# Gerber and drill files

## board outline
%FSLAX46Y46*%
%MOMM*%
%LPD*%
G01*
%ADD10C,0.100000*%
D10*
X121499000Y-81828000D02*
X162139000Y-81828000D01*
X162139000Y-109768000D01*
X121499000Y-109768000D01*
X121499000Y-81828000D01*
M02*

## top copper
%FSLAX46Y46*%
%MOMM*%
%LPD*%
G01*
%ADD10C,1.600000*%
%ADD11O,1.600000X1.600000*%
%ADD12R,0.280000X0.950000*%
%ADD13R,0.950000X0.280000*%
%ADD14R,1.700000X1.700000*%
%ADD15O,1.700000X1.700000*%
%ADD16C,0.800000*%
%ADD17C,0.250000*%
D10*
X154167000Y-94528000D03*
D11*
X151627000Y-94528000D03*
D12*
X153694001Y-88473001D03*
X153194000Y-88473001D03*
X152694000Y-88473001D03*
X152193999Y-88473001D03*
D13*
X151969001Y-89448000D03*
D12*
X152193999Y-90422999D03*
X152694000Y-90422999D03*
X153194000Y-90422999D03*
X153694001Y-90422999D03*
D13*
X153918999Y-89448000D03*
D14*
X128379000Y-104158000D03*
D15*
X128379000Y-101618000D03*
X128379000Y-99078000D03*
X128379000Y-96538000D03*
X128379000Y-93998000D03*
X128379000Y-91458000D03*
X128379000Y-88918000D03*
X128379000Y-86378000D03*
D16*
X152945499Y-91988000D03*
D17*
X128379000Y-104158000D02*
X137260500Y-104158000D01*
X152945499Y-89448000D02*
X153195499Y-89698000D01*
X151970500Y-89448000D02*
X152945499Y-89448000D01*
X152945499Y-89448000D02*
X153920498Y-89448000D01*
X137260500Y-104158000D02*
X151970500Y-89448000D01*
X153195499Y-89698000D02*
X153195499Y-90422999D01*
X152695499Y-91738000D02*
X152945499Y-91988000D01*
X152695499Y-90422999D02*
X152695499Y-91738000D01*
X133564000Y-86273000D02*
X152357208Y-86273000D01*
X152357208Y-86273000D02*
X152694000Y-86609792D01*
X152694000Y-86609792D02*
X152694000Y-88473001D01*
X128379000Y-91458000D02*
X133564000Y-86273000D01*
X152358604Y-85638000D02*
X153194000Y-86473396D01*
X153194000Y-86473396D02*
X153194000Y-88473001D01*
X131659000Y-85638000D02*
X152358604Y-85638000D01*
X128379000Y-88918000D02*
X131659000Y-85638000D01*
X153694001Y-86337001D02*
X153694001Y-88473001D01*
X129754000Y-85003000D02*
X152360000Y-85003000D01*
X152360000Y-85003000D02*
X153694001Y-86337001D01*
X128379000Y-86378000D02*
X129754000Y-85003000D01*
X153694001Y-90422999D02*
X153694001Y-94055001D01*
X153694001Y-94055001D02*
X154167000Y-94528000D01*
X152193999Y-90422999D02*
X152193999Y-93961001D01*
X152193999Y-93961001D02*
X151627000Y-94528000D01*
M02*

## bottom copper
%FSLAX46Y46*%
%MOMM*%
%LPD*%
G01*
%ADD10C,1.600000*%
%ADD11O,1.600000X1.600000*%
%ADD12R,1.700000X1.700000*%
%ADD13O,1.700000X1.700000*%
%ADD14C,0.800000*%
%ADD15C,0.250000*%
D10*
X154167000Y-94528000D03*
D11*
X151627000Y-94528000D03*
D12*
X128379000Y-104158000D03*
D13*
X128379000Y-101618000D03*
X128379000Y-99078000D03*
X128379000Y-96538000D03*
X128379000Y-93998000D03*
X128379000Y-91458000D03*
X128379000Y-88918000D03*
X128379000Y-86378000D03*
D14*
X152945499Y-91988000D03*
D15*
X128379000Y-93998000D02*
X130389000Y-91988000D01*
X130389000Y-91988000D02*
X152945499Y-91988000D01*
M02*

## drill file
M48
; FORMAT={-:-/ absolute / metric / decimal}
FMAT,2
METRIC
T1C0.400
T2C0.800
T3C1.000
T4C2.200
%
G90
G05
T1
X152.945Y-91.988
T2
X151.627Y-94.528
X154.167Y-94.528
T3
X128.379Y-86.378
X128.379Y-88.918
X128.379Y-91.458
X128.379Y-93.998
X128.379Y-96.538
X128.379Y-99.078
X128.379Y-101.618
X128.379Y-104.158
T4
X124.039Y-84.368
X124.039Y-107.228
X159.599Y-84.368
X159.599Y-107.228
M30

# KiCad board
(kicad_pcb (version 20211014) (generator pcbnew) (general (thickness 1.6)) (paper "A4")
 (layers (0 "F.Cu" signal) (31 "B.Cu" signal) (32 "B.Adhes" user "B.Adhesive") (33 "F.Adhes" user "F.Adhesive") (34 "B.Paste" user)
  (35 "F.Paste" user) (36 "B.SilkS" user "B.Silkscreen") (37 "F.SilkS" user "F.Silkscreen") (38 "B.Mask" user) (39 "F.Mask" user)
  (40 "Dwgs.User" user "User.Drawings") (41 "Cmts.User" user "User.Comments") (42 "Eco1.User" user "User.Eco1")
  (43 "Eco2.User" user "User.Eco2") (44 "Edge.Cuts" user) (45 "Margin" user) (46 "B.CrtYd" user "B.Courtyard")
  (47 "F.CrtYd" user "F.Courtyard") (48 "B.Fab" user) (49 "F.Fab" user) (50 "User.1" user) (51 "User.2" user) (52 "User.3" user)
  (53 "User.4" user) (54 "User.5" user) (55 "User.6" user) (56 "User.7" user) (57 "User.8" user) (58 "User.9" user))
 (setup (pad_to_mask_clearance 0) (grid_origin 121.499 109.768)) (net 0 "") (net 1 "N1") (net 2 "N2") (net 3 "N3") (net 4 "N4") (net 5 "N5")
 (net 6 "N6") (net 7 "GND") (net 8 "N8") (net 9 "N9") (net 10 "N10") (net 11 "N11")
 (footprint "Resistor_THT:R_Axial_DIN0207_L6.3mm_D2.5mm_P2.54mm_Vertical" (layer "F.Cu") (at 154.167 94.528 180)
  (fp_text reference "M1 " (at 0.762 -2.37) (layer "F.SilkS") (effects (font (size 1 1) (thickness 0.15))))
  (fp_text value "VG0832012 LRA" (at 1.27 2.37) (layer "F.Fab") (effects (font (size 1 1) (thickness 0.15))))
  (pad "1" thru_hole circle (at 0 0 180) (size 1.6 1.6) (drill 0.8) (layers *.Cu *.Mask) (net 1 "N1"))
  (pad "2" thru_hole oval (at 2.54 0 180) (size 1.6 1.6) (drill 0.8) (layers *.Cu *.Mask) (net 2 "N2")))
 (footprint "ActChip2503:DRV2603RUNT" (layer "F.Cu") (at 152.944 89.448 -90)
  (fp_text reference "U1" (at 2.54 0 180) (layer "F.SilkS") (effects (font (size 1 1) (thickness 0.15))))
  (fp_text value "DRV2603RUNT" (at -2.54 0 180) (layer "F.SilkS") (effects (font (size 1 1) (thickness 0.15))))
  (pad "1" smd rect (at -0.974999 -0.750001) (size 0.28 0.95) (layers "F.Cu" "F.Paste" "F.Mask") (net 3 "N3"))
  (pad "2" smd rect (at -0.974999 -0.25) (size 0.28 0.95) (layers "F.Cu" "F.Paste" "F.Mask") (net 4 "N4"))
  (pad "3" smd rect (at -0.974999 0.25) (size 0.28 0.95) (layers "F.Cu" "F.Paste" "F.Mask") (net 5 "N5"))
  (pad "4" smd rect (at -0.974999 0.750001) (size 0.28 0.95) (layers "F.Cu" "F.Paste" "F.Mask") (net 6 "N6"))
  (pad "5" smd rect (at 0 0.974999 270) (size 0.28 0.95) (layers "F.Cu" "F.Paste" "F.Mask") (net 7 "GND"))
  (pad "6" smd rect (at 0.974999 0.750001) (size 0.28 0.95) (layers "F.Cu" "F.Paste" "F.Mask") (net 2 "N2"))
  (pad "7" smd rect (at 0.974999 0.25) (size 0.28 0.95) (layers "F.Cu" "F.Paste" "F.Mask") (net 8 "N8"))
  (pad "8" smd rect (at 0.974999 -0.25) (size 0.28 0.95) (layers "F.Cu" "F.Paste" "F.Mask") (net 7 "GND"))
  (pad "9" smd rect (at 0.974999 -0.750001) (size 0.28 0.95) (layers "F.Cu" "F.Paste" "F.Mask") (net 1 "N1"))
  (pad "10" smd rect (at 0 -0.974999 270) (size 0.28 0.95) (layers "F.Cu" "F.Paste" "F.Mask") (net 7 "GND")))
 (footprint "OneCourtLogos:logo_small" (layer "F.Cu") (at 141.819 94.528)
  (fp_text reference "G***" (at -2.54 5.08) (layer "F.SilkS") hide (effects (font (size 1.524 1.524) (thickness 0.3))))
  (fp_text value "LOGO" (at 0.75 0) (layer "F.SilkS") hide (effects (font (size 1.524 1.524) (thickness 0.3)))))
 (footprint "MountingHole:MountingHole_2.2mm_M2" (layer "F.Cu") (at 159.599 84.368)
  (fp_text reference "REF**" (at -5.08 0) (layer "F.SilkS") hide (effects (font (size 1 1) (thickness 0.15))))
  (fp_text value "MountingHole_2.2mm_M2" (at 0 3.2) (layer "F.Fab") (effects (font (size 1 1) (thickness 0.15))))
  (pad "" np_thru_hole circle (at 0 0) (size 2.2 2.2) (drill 2.2) (layers *.Cu *.Mask)))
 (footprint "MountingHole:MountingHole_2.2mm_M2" (layer "F.Cu") (at 124.039 107.228)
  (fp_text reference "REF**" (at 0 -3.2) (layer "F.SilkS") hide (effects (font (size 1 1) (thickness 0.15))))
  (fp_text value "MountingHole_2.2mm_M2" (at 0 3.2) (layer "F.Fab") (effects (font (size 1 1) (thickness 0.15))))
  (pad "" np_thru_hole circle (at 0 0) (size 2.2 2.2) (drill 2.2) (layers *.Cu *.Mask)))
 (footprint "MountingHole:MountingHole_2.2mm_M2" (layer "F.Cu") (at 124.039 84.368)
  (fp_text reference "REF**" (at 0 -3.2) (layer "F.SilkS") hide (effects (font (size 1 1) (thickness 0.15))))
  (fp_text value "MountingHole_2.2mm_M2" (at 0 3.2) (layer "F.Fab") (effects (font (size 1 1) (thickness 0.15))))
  (pad "" np_thru_hole circle (at 0 0) (size 2.2 2.2) (drill 2.2) (layers *.Cu *.Mask)))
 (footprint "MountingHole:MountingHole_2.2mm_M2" (layer "F.Cu") (at 159.599 107.228)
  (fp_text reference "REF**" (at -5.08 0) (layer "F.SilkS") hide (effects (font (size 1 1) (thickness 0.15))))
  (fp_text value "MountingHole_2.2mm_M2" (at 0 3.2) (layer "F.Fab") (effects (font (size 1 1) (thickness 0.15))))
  (pad "" np_thru_hole circle (at 0 0) (size 2.2 2.2) (drill 2.2) (layers *.Cu *.Mask)))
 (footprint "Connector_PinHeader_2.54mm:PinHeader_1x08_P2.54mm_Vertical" (layer "F.Cu") (at 128.379 104.158 180)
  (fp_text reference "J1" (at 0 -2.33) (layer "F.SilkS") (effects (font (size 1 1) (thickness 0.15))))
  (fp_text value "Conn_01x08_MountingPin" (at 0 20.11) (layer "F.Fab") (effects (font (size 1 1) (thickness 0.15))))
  (pad "1" thru_hole rect (at 0 0 180) (size 1.7 1.7) (drill 1) (layers *.Cu *.Mask) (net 7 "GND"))
  (pad "2" thru_hole oval (at 0 2.54 180) (size 1.7 1.7) (drill 1) (layers *.Cu *.Mask) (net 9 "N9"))
  (pad "3" thru_hole oval (at 0 5.08 180) (size 1.7 1.7) (drill 1) (layers *.Cu *.Mask) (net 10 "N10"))
  (pad "4" thru_hole oval (at 0 7.62 180) (size 1.7 1.7) (drill 1) (layers *.Cu *.Mask) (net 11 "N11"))
  (pad "5" thru_hole oval (at 0 10.16 180) (size 1.7 1.7) (drill 1) (layers *.Cu *.Mask) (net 8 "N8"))
  (pad "6" thru_hole oval (at 0 12.7 180) (size 1.7 1.7) (drill 1) (layers *.Cu *.Mask) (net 5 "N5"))
  (pad "7" thru_hole oval (at 0 15.24 180) (size 1.7 1.7) (drill 1) (layers *.Cu *.Mask) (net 4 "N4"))
  (pad "8" thru_hole oval (at 0 17.78 180) (size 1.7 1.7) (drill 1) (layers *.Cu *.Mask) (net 3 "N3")))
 (gr_rect (start 121.499 81.828) (end 162.139 109.768) (layer "Edge.Cuts") (width 0.1) (fill none))
 (segment (start 128.379 104.158) (end 137.2605 104.158) (width 0.25) (layer "F.Cu") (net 7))
 (segment (start 152.945499 89.448) (end 153.195499 89.698) (width 0.25) (layer "F.Cu") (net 7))
 (segment (start 151.9705 89.448) (end 152.945499 89.448) (width 0.25) (layer "F.Cu") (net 7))
 (segment (start 152.945499 89.448) (end 153.920498 89.448) (width 0.25) (layer "F.Cu") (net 7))
 (segment (start 137.2605 104.158) (end 151.9705 89.448) (width 0.25) (layer "F.Cu") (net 7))
 (segment (start 153.195499 89.698) (end 153.195499 90.422999) (width 0.25) (layer "F.Cu") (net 7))
 (segment (start 152.695499 91.738) (end 152.945499 91.988) (width 0.25) (layer "F.Cu") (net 8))
 (segment (start 152.695499 90.422999) (end 152.695499 91.738) (width 0.25) (layer "F.Cu") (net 8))
 (via (at 152.945499 91.988) (size 0.8) (drill 0.4) (layers "F.Cu" "B.Cu") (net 8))
 (segment (start 128.379 93.998) (end 130.389 91.988) (width 0.25) (layer "B.Cu") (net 8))
 (segment (start 130.389 91.988) (end 152.945499 91.988) (width 0.25) (layer "B.Cu") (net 8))
 (segment (start 133.564 86.273) (end 152.357208 86.273) (width 0.25) (layer "F.Cu") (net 5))
 (segment (start 152.357208 86.273) (end 152.694 86.609792) (width 0.25) (layer "F.Cu") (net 5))
 (segment (start 152.694 86.609792) (end 152.694 88.473001) (width 0.25) (layer "F.Cu") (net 5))
 (segment (start 128.379 91.458) (end 133.564 86.273) (width 0.25) (layer "F.Cu") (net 5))
 (segment (start 152.358604 85.638) (end 153.194 86.473396) (width 0.25) (layer "F.Cu") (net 4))
 (segment (start 153.194 86.473396) (end 153.194 88.473001) (width 0.25) (layer "F.Cu") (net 4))
 (segment (start 131.659 85.638) (end 152.358604 85.638) (width 0.25) (layer "F.Cu") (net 4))
 (segment (start 128.379 88.918) (end 131.659 85.638) (width 0.25) (layer "F.Cu") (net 4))
 (segment (start 153.694001 86.337001) (end 153.694001 88.473001) (width 0.25) (layer "F.Cu") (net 3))
 (segment (start 129.754 85.003) (end 152.36 85.003) (width 0.25) (layer "F.Cu") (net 3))
 (segment (start 152.36 85.003) (end 153.694001 86.337001) (width 0.25) (layer "F.Cu") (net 3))
 (segment (start 128.379 86.378) (end 129.754 85.003) (width 0.25) (layer "F.Cu") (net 3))
 (segment (start 153.694001 90.422999) (end 153.694001 94.055001) (width 0.25) (layer "F.Cu") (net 1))
 (segment (start 153.694001 94.055001) (end 154.167 94.528) (width 0.25) (layer "F.Cu") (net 1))
 (segment (start 152.193999 90.422999) (end 152.193999 93.961001) (width 0.25) (layer "F.Cu") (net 2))
 (segment (start 152.193999 93.961001) (end 151.627 94.528) (width 0.25) (layer "F.Cu") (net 2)))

